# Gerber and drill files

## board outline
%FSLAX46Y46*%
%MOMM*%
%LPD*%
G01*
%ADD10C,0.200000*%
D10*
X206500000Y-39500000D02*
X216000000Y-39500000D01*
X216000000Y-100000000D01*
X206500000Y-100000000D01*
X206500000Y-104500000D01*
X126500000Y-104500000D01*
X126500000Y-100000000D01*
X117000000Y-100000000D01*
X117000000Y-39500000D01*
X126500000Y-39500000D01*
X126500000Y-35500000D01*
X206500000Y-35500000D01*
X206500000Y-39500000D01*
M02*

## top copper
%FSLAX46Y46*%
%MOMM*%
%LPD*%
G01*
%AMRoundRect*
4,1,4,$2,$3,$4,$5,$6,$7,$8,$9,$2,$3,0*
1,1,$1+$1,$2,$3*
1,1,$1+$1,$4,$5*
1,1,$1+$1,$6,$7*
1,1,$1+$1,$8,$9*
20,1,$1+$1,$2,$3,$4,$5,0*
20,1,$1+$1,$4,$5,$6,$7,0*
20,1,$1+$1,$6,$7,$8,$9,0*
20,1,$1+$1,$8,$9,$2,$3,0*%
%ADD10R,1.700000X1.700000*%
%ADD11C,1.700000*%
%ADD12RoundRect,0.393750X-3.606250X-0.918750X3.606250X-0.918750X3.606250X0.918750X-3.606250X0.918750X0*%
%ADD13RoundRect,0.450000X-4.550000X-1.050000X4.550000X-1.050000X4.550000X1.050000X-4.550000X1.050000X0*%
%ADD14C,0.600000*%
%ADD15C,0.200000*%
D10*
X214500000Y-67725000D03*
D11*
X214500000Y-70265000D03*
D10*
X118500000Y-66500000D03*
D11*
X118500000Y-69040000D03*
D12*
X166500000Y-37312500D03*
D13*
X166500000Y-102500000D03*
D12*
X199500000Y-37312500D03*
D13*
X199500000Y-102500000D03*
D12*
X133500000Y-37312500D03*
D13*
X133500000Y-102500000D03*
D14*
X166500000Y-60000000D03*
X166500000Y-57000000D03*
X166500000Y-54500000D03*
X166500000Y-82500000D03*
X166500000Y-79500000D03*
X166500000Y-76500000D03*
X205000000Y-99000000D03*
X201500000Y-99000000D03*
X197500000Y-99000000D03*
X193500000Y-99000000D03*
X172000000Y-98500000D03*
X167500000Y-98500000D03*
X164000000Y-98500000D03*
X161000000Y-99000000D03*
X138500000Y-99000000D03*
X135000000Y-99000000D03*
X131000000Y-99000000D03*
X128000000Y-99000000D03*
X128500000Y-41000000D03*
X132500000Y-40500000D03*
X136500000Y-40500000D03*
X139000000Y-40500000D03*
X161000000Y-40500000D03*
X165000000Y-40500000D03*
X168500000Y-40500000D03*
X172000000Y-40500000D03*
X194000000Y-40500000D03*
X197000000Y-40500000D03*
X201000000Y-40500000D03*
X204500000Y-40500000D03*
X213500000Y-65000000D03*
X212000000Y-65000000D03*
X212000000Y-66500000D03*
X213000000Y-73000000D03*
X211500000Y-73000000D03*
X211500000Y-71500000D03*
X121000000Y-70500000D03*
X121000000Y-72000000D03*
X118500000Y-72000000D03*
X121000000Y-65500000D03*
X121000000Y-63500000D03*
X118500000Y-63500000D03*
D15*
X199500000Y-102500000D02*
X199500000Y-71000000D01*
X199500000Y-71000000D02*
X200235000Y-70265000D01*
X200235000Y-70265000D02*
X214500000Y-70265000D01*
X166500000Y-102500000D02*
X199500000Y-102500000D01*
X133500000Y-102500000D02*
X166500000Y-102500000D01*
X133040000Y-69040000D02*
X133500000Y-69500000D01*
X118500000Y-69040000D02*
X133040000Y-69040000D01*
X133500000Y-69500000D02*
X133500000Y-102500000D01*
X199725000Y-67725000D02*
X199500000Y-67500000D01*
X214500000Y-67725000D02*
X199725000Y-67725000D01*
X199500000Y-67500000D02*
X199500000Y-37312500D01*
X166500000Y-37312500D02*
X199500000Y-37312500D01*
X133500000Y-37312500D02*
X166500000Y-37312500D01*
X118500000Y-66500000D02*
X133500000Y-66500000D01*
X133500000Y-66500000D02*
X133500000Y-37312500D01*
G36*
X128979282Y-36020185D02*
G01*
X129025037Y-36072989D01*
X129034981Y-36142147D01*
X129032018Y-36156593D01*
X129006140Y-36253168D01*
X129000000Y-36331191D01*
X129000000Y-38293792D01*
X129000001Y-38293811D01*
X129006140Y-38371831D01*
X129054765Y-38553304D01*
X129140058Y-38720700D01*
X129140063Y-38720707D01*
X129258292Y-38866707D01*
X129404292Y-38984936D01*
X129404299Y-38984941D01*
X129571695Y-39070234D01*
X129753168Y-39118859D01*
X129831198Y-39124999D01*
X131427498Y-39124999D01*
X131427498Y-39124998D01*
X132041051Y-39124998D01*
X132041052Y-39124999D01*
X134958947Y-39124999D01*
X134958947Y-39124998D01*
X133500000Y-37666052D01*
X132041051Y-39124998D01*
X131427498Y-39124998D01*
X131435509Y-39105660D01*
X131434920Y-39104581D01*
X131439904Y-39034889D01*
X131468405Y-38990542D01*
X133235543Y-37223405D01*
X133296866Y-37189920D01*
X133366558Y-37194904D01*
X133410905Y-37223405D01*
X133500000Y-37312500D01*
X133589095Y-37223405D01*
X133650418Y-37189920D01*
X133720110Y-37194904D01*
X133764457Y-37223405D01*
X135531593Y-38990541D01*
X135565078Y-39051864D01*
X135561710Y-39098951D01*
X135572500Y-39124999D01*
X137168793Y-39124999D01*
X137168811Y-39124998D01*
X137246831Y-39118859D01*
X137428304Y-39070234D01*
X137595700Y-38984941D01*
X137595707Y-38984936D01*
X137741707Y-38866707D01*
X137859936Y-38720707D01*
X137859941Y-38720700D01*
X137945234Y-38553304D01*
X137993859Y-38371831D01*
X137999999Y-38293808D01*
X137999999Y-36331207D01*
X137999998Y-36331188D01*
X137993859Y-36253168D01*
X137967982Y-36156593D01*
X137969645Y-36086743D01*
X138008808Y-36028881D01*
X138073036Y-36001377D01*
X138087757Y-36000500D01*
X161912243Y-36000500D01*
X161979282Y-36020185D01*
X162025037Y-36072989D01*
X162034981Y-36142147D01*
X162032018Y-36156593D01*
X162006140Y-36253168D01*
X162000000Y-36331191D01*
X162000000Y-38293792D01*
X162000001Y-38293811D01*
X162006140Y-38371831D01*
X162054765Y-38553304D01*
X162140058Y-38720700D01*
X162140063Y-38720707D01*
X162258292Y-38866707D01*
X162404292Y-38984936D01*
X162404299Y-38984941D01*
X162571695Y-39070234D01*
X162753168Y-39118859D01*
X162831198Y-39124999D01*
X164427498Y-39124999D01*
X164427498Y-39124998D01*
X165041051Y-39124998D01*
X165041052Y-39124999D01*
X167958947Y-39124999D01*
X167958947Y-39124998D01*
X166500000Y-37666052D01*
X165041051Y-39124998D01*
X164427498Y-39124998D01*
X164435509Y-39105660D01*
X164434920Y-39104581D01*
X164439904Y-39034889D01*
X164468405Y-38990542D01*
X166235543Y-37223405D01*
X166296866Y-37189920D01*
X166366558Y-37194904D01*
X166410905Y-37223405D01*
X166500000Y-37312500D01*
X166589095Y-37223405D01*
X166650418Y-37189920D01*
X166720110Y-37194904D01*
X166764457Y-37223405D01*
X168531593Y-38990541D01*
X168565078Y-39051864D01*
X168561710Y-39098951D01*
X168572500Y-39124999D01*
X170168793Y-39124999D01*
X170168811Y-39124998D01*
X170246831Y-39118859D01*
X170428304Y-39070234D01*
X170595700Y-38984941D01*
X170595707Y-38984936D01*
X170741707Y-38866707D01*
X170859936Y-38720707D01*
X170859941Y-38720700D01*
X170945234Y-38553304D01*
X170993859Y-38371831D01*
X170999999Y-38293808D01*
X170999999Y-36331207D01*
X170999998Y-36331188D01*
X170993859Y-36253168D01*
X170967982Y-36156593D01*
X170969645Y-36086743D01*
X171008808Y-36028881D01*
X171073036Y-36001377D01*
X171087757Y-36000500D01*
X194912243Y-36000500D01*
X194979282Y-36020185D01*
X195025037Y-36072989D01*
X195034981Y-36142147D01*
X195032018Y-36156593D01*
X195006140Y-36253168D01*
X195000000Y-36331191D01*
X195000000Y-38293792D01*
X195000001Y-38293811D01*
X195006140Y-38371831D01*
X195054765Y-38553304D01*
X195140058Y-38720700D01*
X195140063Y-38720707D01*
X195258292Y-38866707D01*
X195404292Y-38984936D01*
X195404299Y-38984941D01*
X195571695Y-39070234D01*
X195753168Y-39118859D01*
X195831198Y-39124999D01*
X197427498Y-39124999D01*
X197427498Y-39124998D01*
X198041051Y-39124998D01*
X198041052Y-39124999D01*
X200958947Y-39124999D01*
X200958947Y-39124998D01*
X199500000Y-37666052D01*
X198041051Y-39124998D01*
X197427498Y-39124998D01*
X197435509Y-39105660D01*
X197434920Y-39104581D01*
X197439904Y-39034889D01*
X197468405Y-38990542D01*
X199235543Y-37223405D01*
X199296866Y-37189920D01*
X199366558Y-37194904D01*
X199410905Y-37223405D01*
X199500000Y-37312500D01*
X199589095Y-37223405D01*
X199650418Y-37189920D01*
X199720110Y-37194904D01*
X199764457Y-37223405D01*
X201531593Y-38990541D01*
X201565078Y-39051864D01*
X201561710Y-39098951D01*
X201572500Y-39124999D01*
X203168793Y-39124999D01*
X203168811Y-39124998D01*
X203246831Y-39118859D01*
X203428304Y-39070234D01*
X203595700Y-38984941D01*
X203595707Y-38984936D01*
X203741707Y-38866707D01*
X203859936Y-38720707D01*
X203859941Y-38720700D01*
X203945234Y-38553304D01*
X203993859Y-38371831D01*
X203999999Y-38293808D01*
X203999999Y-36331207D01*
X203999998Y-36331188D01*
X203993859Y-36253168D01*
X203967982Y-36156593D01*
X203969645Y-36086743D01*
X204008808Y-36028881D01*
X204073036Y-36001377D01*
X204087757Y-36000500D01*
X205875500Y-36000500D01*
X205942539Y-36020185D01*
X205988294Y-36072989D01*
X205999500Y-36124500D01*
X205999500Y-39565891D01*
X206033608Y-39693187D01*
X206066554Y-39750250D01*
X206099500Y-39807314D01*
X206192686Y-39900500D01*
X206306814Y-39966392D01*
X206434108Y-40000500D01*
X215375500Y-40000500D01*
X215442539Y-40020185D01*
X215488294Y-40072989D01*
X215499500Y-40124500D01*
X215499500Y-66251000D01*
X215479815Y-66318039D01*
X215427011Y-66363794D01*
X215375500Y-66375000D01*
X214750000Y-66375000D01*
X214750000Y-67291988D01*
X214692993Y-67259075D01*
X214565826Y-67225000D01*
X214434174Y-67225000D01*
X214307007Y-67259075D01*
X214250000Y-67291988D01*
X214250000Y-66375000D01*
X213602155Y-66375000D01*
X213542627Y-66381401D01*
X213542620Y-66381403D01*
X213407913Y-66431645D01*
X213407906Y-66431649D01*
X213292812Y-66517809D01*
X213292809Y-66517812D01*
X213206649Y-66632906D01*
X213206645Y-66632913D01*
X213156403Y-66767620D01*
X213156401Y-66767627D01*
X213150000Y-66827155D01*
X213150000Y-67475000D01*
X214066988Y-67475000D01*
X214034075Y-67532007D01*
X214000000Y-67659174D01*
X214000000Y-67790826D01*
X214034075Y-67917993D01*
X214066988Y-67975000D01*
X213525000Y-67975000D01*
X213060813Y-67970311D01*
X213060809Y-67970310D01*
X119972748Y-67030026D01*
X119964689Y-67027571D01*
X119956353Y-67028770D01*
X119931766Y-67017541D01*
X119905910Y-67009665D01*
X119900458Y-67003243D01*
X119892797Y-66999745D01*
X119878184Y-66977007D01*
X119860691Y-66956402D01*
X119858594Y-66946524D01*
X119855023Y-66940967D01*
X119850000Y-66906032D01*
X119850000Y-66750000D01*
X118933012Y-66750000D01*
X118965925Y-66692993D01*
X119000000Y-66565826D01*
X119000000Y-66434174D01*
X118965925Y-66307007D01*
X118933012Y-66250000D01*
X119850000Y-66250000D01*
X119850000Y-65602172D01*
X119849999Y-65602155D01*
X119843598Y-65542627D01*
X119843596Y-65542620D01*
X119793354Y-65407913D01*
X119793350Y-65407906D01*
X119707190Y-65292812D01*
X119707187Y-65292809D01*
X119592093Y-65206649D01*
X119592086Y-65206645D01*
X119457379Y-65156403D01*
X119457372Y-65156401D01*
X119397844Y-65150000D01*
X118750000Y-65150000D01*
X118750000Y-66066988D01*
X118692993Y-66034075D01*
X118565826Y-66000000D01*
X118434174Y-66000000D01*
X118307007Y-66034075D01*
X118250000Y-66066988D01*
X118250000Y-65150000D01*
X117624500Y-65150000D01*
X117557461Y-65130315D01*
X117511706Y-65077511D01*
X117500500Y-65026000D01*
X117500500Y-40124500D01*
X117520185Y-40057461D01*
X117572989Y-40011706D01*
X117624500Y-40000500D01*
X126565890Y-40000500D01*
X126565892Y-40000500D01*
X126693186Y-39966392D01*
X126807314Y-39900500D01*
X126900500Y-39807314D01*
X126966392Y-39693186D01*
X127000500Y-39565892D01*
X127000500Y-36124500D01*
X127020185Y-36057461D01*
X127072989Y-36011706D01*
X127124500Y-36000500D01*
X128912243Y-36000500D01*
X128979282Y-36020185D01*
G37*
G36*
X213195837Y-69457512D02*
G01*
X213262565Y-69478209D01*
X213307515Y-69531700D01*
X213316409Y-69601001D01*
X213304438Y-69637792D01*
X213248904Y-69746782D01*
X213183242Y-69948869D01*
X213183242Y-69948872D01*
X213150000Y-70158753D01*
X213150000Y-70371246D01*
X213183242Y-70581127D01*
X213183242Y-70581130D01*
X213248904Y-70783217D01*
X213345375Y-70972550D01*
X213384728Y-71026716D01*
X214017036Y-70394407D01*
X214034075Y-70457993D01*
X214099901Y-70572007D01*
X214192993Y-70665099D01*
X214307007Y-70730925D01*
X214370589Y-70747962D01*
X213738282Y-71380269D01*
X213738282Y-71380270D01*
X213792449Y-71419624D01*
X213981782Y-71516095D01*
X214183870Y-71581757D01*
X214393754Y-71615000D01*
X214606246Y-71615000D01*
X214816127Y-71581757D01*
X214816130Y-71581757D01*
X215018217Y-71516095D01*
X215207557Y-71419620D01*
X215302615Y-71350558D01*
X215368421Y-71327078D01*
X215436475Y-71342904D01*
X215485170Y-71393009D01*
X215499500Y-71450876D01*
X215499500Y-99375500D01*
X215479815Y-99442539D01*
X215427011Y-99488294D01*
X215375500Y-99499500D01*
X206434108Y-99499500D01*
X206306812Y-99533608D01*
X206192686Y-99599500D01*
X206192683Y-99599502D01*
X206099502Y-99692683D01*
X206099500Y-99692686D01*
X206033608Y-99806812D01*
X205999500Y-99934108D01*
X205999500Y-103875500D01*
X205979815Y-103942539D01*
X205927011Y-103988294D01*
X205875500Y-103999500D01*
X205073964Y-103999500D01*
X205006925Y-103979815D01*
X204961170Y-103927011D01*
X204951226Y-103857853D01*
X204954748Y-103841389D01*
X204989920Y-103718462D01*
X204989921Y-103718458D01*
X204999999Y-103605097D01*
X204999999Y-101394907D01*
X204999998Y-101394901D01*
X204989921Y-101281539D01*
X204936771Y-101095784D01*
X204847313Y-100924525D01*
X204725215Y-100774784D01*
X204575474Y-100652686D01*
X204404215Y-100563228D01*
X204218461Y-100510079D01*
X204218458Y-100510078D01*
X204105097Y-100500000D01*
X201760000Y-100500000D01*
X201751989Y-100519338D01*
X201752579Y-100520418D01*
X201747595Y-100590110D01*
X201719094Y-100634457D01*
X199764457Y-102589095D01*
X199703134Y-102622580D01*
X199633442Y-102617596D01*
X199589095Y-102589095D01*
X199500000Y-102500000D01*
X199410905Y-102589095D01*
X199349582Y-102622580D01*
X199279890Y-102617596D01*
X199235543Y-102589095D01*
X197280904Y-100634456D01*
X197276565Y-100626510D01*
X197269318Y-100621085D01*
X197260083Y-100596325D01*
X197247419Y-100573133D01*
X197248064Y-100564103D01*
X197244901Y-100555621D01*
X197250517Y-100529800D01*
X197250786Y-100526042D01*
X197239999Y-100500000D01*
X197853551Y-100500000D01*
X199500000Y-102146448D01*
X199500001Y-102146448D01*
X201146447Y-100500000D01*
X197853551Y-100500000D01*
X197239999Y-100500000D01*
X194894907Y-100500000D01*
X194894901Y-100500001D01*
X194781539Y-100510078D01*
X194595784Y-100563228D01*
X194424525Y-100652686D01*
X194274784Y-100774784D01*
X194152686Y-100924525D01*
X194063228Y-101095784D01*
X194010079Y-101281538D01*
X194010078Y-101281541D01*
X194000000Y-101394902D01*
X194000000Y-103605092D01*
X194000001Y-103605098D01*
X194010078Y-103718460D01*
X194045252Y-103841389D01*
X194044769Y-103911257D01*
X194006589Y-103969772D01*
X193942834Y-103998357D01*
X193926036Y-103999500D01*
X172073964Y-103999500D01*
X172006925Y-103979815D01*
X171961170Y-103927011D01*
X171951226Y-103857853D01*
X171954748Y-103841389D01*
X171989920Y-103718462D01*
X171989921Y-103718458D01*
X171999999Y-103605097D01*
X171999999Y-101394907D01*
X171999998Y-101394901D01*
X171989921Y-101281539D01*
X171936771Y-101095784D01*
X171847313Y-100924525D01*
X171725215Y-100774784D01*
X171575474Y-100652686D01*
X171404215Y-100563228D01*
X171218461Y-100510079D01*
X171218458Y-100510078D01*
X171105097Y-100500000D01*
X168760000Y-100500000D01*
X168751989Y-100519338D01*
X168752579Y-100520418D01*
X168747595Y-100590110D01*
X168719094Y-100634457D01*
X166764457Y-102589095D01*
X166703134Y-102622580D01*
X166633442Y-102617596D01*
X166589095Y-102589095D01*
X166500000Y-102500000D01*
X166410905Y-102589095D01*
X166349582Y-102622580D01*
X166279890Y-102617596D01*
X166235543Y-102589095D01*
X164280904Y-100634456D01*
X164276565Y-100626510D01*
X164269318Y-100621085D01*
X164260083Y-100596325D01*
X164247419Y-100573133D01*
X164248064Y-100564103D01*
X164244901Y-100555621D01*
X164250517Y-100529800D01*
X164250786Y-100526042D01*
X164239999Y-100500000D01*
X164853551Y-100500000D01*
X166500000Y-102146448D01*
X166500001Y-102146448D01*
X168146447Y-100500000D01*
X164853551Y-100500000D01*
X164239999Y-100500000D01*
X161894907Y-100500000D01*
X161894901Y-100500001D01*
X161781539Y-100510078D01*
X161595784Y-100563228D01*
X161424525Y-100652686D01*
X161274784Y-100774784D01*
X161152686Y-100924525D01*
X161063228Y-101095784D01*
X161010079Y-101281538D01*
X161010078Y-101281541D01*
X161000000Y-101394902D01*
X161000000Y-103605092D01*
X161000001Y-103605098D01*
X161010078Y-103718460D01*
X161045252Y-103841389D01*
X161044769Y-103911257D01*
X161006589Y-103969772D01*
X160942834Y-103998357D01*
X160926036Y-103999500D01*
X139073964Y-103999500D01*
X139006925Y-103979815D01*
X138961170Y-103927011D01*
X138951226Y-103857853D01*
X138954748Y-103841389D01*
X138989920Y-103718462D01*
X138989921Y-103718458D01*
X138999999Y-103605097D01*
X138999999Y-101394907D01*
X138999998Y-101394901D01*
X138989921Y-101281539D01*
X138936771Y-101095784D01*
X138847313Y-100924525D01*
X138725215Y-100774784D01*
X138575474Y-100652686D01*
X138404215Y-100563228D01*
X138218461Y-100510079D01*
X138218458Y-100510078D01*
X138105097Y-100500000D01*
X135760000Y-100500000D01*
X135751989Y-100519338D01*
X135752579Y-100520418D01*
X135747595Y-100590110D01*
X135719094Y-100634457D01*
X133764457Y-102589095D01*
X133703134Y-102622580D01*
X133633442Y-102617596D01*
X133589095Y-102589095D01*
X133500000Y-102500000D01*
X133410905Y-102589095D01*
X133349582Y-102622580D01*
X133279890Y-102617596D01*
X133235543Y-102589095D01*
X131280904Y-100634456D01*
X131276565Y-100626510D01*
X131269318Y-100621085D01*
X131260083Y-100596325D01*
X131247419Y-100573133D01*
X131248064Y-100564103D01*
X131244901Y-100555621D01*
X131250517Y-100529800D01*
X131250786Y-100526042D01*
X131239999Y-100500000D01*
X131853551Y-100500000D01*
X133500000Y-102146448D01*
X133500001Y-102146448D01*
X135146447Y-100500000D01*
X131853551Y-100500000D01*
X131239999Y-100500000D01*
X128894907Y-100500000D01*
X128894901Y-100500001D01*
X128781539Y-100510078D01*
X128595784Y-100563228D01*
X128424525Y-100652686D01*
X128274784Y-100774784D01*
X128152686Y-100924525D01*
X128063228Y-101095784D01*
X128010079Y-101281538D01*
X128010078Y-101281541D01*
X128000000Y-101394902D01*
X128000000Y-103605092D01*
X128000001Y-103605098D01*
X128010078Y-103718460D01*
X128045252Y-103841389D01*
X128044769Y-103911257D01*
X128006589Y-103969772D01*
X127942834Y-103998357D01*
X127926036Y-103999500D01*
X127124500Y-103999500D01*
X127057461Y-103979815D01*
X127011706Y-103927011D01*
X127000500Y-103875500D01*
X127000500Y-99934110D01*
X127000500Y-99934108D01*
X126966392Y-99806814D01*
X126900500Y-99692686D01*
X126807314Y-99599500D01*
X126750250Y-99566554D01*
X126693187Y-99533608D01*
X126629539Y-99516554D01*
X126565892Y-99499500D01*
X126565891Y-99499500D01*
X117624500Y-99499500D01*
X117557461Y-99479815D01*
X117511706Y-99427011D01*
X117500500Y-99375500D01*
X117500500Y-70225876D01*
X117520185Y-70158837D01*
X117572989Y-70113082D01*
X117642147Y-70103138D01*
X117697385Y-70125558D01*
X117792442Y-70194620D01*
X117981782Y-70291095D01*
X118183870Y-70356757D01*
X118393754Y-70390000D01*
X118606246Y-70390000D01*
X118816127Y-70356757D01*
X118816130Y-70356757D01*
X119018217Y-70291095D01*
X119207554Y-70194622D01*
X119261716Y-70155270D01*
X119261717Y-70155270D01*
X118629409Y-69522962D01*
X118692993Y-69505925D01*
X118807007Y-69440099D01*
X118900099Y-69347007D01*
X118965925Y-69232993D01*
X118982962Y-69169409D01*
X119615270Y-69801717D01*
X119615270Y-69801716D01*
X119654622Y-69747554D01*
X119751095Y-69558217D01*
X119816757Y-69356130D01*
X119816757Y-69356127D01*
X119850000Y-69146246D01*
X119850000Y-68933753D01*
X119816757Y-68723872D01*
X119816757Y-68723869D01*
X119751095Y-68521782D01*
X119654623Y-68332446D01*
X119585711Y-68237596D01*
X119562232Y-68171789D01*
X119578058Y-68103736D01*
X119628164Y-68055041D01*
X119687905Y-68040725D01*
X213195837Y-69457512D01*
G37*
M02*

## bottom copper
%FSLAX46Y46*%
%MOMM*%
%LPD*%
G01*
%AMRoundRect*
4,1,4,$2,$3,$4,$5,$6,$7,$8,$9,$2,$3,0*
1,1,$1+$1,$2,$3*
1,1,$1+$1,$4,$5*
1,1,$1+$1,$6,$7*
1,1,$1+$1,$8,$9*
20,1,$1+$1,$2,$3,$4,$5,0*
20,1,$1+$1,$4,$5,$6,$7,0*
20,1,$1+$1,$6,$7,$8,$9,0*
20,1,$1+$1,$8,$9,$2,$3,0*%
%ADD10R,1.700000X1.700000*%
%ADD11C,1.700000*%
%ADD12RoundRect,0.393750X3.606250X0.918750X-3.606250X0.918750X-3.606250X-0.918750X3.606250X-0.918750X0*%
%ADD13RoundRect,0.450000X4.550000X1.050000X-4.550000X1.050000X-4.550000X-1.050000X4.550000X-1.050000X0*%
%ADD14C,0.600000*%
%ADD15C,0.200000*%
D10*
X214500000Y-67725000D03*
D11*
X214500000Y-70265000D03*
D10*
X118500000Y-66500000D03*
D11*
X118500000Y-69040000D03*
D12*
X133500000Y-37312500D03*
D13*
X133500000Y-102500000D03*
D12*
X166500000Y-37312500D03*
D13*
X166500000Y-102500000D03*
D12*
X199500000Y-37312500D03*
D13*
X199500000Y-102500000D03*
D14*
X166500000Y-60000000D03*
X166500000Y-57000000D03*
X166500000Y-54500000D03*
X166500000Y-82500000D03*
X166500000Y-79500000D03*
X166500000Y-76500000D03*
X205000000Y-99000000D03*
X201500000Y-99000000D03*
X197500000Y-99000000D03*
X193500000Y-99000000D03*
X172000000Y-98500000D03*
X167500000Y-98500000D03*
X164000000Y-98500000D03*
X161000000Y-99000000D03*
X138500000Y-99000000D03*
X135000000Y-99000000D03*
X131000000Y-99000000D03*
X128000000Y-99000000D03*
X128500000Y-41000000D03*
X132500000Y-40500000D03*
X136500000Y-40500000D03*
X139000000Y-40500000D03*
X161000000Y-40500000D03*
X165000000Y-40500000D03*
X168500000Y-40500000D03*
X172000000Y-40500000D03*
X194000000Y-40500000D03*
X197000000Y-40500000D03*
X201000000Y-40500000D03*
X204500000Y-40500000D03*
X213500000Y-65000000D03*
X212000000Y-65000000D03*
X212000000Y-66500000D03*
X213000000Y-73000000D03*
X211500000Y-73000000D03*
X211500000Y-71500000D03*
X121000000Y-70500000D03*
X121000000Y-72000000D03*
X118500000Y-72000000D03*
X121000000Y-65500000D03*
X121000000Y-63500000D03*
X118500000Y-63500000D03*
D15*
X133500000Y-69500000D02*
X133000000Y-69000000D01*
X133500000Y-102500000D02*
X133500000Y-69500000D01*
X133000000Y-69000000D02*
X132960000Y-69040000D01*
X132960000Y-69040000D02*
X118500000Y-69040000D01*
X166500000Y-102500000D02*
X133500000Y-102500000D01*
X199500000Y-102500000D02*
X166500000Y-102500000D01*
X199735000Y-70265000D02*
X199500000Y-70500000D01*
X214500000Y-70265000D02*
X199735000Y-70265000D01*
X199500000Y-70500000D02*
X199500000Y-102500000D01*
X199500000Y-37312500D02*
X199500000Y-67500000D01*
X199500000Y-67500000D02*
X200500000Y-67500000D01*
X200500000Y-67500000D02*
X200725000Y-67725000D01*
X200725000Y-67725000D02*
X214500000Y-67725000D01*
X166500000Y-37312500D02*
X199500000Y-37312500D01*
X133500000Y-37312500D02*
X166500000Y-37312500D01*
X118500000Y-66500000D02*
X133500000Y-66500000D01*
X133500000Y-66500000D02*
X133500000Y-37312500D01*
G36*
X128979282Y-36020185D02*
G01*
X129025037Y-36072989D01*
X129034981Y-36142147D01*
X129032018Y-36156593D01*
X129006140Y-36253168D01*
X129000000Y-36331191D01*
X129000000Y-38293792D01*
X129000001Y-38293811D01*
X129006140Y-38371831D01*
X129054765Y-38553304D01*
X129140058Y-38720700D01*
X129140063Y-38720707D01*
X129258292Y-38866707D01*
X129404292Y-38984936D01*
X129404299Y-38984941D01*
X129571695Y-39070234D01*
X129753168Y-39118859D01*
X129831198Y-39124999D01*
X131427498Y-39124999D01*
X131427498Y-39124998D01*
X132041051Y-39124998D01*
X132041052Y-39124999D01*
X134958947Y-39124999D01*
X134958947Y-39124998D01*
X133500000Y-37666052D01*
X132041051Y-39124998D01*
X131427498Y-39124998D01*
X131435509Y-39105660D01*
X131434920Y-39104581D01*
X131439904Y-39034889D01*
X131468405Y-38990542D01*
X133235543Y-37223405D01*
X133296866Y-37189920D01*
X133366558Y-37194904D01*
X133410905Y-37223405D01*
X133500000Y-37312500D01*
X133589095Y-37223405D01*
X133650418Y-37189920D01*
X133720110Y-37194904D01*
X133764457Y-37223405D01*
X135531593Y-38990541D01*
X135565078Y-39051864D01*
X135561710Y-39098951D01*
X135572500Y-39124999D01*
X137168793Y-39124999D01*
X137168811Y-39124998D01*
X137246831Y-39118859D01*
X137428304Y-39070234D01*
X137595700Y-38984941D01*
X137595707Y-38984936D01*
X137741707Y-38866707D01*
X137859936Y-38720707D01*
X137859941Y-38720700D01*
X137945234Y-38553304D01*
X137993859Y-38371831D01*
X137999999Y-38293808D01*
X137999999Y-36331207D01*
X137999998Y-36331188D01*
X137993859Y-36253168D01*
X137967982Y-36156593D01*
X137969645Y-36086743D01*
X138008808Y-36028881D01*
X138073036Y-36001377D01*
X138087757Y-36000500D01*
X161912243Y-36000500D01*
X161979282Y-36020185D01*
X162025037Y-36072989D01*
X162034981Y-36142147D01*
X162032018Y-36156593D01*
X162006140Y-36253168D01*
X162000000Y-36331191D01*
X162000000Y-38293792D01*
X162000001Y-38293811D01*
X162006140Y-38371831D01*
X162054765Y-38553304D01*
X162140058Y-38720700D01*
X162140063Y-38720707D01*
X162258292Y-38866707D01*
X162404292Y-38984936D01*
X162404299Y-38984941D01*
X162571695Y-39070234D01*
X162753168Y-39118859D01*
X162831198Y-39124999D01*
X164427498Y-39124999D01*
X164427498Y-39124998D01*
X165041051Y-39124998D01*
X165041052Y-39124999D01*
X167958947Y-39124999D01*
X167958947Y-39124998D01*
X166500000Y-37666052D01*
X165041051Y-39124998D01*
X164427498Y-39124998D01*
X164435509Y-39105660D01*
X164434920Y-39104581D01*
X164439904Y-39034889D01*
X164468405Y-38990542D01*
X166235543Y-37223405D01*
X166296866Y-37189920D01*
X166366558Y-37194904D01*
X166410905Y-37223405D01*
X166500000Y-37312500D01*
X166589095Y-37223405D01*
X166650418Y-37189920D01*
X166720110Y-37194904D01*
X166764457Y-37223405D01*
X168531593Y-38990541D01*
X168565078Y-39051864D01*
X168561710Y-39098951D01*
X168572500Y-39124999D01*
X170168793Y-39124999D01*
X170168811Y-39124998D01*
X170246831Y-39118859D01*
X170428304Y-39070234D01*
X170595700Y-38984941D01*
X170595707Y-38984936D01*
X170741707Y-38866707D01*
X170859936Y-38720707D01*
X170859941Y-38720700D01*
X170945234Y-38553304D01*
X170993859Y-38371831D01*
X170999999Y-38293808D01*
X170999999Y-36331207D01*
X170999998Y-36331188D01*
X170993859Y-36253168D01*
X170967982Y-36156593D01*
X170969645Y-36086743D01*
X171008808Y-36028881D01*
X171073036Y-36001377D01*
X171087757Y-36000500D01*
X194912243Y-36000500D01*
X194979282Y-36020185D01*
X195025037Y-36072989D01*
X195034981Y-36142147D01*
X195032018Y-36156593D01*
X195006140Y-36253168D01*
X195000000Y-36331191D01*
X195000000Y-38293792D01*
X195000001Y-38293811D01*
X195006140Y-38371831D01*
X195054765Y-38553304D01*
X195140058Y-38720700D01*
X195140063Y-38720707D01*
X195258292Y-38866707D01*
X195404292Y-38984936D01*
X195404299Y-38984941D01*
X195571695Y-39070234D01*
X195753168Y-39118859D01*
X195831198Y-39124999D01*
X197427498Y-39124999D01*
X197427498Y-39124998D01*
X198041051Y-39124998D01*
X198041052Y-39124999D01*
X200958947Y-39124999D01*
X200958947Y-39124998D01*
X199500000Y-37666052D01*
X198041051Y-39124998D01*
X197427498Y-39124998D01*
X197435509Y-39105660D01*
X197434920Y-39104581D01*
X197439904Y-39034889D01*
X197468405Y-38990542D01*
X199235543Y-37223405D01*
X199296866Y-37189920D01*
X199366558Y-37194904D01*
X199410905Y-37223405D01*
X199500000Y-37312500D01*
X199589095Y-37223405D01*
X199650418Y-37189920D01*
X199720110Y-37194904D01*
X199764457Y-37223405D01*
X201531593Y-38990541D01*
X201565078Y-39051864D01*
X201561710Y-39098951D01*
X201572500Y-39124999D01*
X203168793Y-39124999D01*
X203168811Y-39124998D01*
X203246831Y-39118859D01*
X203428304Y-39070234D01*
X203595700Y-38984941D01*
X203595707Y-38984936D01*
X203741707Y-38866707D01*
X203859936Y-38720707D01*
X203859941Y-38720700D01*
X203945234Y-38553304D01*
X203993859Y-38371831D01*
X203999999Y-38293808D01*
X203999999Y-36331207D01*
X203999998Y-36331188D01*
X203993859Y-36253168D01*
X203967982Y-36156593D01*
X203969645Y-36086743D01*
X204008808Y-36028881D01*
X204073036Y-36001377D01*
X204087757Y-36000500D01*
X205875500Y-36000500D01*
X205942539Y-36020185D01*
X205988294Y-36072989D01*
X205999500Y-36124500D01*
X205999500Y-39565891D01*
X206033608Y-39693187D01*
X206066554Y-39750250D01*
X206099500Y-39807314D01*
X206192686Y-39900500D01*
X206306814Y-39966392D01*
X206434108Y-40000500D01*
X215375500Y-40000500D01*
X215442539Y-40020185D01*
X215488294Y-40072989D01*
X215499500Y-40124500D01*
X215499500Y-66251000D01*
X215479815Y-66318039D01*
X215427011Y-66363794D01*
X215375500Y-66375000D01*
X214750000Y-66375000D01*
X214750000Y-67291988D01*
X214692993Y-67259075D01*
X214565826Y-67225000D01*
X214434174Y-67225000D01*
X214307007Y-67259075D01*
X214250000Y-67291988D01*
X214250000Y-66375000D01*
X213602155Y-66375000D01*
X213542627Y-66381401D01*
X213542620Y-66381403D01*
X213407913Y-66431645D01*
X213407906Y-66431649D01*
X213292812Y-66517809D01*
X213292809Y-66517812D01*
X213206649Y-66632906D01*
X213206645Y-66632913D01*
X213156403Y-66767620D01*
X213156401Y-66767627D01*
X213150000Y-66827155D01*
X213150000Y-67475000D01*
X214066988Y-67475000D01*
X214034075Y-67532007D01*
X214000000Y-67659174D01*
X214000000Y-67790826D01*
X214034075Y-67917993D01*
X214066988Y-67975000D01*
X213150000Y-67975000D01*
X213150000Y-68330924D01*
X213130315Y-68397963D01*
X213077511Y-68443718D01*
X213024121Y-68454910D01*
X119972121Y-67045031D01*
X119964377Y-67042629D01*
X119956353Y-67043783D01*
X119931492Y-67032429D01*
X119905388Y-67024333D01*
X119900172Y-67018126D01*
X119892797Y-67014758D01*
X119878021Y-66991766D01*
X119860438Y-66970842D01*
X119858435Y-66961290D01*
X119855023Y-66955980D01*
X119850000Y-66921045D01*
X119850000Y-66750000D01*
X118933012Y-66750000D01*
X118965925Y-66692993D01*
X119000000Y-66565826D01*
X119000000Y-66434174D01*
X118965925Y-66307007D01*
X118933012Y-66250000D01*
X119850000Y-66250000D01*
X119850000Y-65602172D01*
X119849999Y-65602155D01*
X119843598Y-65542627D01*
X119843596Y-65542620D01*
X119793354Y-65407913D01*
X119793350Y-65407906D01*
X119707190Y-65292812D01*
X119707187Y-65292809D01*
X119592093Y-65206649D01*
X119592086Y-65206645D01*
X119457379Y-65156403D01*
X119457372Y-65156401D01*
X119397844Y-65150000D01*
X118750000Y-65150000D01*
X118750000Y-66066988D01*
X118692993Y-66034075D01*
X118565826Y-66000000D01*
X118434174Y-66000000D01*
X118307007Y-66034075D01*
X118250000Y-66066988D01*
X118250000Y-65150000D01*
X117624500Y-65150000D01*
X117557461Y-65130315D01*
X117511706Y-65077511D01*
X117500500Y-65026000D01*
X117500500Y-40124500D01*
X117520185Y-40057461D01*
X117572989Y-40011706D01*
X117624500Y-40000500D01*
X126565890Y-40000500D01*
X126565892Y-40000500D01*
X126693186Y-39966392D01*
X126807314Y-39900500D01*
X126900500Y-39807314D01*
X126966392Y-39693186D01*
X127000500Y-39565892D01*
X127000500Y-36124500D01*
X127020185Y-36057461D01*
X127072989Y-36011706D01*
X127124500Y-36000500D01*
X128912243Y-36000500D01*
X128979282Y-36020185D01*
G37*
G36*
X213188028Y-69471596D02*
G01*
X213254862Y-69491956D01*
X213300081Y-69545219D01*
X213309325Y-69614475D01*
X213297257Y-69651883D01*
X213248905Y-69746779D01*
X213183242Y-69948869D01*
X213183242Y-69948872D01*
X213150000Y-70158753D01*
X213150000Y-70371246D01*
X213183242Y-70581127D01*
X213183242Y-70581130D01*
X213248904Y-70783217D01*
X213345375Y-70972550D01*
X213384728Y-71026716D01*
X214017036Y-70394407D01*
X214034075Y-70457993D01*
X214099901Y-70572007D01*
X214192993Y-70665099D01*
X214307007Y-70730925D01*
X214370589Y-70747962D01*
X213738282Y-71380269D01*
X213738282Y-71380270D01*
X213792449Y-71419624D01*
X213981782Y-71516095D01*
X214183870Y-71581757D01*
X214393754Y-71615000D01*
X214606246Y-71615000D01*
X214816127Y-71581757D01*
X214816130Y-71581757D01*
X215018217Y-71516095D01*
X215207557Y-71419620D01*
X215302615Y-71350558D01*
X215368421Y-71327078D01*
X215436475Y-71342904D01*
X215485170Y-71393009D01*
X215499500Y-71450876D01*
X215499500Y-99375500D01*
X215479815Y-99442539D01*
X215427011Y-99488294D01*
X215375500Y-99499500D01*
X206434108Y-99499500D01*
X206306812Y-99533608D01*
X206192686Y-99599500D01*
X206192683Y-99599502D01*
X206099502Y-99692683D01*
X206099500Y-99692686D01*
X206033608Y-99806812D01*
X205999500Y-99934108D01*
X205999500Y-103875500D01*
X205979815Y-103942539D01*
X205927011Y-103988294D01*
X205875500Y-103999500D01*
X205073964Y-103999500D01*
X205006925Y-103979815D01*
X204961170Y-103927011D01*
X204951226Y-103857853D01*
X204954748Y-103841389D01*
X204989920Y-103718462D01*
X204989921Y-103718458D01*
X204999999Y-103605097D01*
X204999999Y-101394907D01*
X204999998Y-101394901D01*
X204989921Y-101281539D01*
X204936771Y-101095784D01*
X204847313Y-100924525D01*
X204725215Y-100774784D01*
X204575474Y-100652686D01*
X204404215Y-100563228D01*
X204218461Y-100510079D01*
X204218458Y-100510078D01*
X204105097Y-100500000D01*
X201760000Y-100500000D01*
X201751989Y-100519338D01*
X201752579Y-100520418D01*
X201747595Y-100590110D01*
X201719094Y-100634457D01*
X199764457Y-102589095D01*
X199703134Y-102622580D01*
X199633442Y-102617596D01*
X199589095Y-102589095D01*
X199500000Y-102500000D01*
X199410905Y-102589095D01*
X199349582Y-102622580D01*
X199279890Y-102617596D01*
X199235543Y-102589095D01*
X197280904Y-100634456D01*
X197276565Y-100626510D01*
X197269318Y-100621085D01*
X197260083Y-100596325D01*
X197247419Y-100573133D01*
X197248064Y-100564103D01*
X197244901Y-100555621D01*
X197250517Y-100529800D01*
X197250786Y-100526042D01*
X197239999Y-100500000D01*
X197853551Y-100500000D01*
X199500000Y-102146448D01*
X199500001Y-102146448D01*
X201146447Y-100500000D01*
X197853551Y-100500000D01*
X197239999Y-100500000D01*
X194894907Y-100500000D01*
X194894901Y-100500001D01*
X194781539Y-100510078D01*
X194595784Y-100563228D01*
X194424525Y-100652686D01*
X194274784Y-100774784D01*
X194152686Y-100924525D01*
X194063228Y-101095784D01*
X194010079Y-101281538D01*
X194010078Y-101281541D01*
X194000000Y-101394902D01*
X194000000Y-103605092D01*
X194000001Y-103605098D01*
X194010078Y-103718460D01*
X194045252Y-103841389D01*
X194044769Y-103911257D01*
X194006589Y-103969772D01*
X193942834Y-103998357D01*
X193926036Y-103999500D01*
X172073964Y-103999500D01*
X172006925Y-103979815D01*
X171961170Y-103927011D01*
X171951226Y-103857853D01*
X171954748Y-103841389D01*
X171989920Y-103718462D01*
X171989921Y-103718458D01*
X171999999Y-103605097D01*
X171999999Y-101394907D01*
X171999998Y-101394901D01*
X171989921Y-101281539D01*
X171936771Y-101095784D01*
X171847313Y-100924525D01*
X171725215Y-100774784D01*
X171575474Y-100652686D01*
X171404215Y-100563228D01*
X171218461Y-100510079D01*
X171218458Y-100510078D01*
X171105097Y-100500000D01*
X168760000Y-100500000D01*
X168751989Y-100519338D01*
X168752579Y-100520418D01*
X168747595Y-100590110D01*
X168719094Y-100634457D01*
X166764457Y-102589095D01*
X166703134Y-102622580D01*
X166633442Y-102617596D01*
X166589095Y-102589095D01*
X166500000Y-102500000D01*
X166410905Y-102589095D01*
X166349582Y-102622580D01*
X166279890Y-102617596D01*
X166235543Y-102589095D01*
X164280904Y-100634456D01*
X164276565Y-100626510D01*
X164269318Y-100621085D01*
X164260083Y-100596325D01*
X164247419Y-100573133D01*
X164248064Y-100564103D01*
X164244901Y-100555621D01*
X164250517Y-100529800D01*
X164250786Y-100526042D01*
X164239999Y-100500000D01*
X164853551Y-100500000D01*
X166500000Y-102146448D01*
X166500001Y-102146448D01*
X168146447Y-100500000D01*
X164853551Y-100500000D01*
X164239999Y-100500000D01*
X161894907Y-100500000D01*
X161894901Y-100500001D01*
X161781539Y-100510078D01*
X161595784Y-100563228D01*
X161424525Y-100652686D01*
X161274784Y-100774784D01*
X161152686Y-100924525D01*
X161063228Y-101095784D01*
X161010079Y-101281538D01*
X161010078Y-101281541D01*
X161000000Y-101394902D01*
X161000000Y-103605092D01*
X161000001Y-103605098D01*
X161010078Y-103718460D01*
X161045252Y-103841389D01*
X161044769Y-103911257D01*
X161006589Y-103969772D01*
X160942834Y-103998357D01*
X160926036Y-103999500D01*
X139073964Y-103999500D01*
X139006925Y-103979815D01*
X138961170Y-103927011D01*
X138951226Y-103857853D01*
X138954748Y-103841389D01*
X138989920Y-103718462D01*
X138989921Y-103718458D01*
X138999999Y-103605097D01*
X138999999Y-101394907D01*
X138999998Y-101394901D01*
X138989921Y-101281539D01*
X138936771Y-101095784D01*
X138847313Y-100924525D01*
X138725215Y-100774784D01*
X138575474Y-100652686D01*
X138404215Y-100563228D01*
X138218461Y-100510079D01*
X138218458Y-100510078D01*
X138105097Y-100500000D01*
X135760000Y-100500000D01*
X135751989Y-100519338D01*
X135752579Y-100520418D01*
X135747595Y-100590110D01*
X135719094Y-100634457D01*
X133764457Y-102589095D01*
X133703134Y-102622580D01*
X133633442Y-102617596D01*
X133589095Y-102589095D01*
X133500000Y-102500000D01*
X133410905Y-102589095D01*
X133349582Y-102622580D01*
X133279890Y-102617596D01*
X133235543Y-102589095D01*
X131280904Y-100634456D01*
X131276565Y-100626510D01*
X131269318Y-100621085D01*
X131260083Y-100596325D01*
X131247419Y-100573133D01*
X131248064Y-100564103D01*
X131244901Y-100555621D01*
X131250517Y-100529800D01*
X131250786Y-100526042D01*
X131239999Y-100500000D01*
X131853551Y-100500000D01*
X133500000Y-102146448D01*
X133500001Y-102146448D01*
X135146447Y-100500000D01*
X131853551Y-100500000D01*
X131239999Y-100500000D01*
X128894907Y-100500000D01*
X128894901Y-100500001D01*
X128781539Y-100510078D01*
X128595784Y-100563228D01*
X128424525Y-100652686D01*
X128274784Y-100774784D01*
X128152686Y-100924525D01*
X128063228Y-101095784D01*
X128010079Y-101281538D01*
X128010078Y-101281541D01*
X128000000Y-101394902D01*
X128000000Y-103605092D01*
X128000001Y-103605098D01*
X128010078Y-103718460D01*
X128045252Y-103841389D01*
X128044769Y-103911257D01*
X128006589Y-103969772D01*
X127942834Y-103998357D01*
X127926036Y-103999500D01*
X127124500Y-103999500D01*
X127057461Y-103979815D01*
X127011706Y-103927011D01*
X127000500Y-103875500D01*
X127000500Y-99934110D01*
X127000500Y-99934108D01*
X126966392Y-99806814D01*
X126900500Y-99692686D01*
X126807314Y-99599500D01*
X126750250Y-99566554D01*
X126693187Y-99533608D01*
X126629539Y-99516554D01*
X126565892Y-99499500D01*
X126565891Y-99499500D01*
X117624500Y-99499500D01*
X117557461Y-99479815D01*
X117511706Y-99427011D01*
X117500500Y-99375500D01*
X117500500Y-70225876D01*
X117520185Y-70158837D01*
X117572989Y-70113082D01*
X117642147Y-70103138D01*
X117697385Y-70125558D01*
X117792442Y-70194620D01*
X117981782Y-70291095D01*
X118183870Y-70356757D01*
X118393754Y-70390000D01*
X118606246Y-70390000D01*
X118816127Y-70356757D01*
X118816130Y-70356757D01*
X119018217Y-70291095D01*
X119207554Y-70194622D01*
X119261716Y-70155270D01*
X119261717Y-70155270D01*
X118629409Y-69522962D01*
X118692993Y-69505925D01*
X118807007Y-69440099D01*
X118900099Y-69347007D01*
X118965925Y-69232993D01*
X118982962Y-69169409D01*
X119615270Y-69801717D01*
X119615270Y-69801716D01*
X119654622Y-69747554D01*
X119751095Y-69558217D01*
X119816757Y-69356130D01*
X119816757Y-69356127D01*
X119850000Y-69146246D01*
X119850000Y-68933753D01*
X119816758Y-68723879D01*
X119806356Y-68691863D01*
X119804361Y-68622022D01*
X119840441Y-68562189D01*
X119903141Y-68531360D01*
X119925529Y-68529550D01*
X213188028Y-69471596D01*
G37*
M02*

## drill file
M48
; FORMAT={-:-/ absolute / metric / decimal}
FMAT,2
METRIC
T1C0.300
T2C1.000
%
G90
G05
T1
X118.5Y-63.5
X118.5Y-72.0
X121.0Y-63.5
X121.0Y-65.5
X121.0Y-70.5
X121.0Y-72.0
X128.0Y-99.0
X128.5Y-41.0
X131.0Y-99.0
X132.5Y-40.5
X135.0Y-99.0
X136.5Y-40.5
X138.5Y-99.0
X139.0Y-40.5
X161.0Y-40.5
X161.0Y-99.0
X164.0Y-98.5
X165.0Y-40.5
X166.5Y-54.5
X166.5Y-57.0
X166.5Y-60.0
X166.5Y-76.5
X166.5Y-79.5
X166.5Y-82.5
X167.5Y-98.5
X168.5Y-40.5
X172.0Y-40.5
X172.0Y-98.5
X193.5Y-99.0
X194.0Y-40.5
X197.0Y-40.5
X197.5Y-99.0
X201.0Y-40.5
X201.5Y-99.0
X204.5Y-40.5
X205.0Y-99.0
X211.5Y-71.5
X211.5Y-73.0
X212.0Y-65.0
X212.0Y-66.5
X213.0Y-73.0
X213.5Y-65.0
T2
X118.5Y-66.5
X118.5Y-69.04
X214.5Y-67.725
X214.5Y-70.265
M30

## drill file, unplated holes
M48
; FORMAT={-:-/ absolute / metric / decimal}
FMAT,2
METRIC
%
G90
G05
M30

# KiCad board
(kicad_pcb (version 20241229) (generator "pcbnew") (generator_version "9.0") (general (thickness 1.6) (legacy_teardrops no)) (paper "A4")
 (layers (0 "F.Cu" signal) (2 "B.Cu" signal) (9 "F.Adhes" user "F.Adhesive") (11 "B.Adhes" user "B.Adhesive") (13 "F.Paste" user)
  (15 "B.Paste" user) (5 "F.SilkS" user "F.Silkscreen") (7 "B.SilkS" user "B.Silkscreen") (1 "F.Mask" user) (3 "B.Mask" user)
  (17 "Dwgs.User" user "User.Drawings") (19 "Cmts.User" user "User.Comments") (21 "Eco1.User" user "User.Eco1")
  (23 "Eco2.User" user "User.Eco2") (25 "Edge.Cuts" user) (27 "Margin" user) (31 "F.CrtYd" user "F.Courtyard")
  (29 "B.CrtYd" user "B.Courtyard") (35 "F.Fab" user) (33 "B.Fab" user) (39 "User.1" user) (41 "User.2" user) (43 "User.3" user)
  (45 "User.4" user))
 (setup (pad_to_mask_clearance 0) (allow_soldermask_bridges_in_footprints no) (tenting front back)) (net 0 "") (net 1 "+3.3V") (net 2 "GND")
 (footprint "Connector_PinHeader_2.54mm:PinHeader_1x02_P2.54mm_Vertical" (layer "F.Cu") (at 214.5 67.725)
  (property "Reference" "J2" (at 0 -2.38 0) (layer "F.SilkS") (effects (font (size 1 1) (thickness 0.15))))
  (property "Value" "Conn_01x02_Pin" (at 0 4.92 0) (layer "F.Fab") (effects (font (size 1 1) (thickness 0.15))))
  (pad "1" thru_hole rect (at 0 0) (size 1.7 1.7) (drill 1) (layers "*.Cu" "*.Mask") (remove_unused_layers no) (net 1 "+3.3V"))
  (pad "2" thru_hole circle (at 0 2.54) (size 1.7 1.7) (drill 1) (layers "*.Cu" "*.Mask") (remove_unused_layers no) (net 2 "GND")))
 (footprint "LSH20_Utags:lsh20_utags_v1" (layer "F.Cu") (at 166.5 70)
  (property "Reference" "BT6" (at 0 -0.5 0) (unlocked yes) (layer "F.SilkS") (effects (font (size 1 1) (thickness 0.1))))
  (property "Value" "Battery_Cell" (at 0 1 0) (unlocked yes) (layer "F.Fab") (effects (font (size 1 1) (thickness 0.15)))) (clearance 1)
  (pad "1" smd roundrect (at 0 -32.6875) (size 8 2.625) (layers "F.Cu" "F.Mask" "F.Paste") (roundrect_rratio 0.15) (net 1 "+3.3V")
   (thermal_bridge_angle 45))
  (pad "2" smd roundrect (at 0 32.5) (size 10 3) (layers "F.Cu" "F.Mask" "F.Paste") (roundrect_rratio 0.15) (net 2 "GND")
   (thermal_bridge_angle 45)))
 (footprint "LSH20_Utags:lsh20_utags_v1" (layer "F.Cu") (at 199.5 70)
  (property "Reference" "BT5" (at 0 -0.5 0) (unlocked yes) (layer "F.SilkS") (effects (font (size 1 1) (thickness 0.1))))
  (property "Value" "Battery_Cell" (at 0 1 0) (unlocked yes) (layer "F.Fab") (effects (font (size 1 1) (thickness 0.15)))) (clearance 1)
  (pad "1" smd roundrect (at 0 -32.6875) (size 8 2.625) (layers "F.Cu" "F.Mask" "F.Paste") (roundrect_rratio 0.15) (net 1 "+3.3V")
   (thermal_bridge_angle 45))
  (pad "2" smd roundrect (at 0 32.5) (size 10 3) (layers "F.Cu" "F.Mask" "F.Paste") (roundrect_rratio 0.15) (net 2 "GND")
   (thermal_bridge_angle 45)))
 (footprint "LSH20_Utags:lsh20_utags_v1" (layer "F.Cu") (at 133.5 70)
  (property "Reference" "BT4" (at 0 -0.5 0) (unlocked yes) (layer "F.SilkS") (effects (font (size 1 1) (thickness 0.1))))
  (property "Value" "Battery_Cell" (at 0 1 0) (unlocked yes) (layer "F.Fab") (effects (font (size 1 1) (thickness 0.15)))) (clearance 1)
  (pad "1" smd roundrect (at 0 -32.6875) (size 8 2.625) (layers "F.Cu" "F.Mask" "F.Paste") (roundrect_rratio 0.15) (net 1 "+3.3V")
   (thermal_bridge_angle 45))
  (pad "2" smd roundrect (at 0 32.5) (size 10 3) (layers "F.Cu" "F.Mask" "F.Paste") (roundrect_rratio 0.15) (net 2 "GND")
   (thermal_bridge_angle 45)))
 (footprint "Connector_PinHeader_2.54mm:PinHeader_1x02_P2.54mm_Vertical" (layer "F.Cu") (at 118.5 66.5)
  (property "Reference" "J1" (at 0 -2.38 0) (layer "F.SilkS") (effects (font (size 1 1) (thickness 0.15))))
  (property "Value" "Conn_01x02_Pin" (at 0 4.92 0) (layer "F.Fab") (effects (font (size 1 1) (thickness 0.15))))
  (pad "1" thru_hole rect (at 0 0) (size 1.7 1.7) (drill 1) (layers "*.Cu" "*.Mask") (remove_unused_layers no) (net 1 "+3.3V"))
  (pad "2" thru_hole circle (at 0 2.54) (size 1.7 1.7) (drill 1) (layers "*.Cu" "*.Mask") (remove_unused_layers no) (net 2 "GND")))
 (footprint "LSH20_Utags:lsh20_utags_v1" (layer "B.Cu") (at 166.5 70 180)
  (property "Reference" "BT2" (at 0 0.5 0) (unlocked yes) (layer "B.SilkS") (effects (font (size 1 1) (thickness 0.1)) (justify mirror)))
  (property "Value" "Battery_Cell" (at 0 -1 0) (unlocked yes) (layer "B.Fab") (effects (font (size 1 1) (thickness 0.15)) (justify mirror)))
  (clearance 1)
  (pad "1" smd roundrect (at 0 32.6875 180) (size 8 2.625) (layers "B.Cu" "B.Mask" "B.Paste") (roundrect_rratio 0.15) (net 1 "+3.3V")
   (thermal_bridge_angle 45))
  (pad "2" smd roundrect (at 0 -32.5 180) (size 10 3) (layers "B.Cu" "B.Mask" "B.Paste") (roundrect_rratio 0.15) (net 2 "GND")
   (thermal_bridge_angle 45)))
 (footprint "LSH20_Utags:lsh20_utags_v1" (layer "B.Cu") (at 199.5 70 180)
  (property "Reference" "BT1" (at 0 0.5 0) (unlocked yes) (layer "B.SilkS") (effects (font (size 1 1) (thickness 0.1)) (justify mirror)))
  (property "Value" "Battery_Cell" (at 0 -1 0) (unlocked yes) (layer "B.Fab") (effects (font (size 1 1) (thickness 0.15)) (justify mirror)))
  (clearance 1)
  (pad "1" smd roundrect (at 0 32.6875 180) (size 8 2.625) (layers "B.Cu" "B.Mask" "B.Paste") (roundrect_rratio 0.15) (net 1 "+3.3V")
   (thermal_bridge_angle 45))
  (pad "2" smd roundrect (at 0 -32.5 180) (size 10 3) (layers "B.Cu" "B.Mask" "B.Paste") (roundrect_rratio 0.15) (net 2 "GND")
   (thermal_bridge_angle 45)))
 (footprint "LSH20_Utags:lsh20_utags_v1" (layer "B.Cu") (at 133.5 70 180)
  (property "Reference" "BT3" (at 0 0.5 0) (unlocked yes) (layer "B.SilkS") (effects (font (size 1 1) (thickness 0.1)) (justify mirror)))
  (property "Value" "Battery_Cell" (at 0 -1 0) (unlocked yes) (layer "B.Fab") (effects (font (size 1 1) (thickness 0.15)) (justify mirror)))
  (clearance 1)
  (pad "1" smd roundrect (at 0 32.6875 180) (size 8 2.625) (layers "B.Cu" "B.Mask" "B.Paste") (roundrect_rratio 0.15) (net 1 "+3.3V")
   (thermal_bridge_angle 45))
  (pad "2" smd roundrect (at 0 -32.5 180) (size 10 3) (layers "B.Cu" "B.Mask" "B.Paste") (roundrect_rratio 0.15) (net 2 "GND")
   (thermal_bridge_angle 45)))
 (gr_poly
  (pts (xy 117 39.5) (xy 126.5 39.5) (xy 126.5 35.5) (xy 206.5 35.5) (xy 206.5 39.5) (xy 216 39.5) (xy 216 100) (xy 206.5 100)
   (xy 206.5 104.5) (xy 126.5 104.5) (xy 126.5 100) (xy 117 100))
  (stroke (width 0.2) (type solid)) (fill no) (layer "Edge.Cuts"))
 (segment (start 166.5 37.3125) (end 199.5 37.3125) (width 0.2) (layer "F.Cu") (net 1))
 (segment (start 133.5 37.3125) (end 166.5 37.3125) (width 0.2) (layer "F.Cu") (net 1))
 (segment (start 199.5 67.5) (end 199.5 37.3125) (width 0.2) (layer "F.Cu") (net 1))
 (segment (start 118.5 66.5) (end 133.5 66.5) (width 0.2) (layer "F.Cu") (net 1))
 (segment (start 133.5 66.5) (end 133.5 37.3125) (width 0.2) (layer "F.Cu") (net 1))
 (segment (start 214.5 67.725) (end 199.725 67.725) (width 0.2) (layer "F.Cu") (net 1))
 (segment (start 199.725 67.725) (end 199.5 67.5) (width 0.2) (layer "F.Cu") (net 1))
 (via (at 136.5 40.5) (size 0.6) (drill 0.3) (layers "F.Cu" "B.Cu") (free yes) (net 1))
 (via (at 165 40.5) (size 0.6) (drill 0.3) (layers "F.Cu" "B.Cu") (free yes) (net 1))
 (via (at 213.5 65) (size 0.6) (drill 0.3) (layers "F.Cu" "B.Cu") (free yes) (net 1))
 (via (at 197 40.5) (size 0.6) (drill 0.3) (layers "F.Cu" "B.Cu") (free yes) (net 1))
 (via (at 212 65) (size 0.6) (drill 0.3) (layers "F.Cu" "B.Cu") (free yes) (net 1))
 (via (at 168.5 40.5) (size 0.6) (drill 0.3) (layers "F.Cu" "B.Cu") (free yes) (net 1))
 (via (at 121 63.5) (size 0.6) (drill 0.3) (layers "F.Cu" "B.Cu") (free yes) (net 1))
 (via (at 172 40.5) (size 0.6) (drill 0.3) (layers "F.Cu" "B.Cu") (free yes) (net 1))
 (via (at 201 40.5) (size 0.6) (drill 0.3) (layers "F.Cu" "B.Cu") (free yes) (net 1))
 (via (at 166.5 60) (size 0.6) (drill 0.3) (layers "F.Cu" "B.Cu") (free yes) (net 1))
 (via (at 132.5 40.5) (size 0.6) (drill 0.3) (layers "F.Cu" "B.Cu") (free yes) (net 1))
 (via (at 166.5 57) (size 0.6) (drill 0.3) (layers "F.Cu" "B.Cu") (free yes) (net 1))
 (via (at 212 66.5) (size 0.6) (drill 0.3) (layers "F.Cu" "B.Cu") (free yes) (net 1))
 (via (at 194 40.5) (size 0.6) (drill 0.3) (layers "F.Cu" "B.Cu") (free yes) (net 1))
 (via (at 128.5 41) (size 0.6) (drill 0.3) (layers "F.Cu" "B.Cu") (free yes) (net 1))
 (via (at 204.5 40.5) (size 0.6) (drill 0.3) (layers "F.Cu" "B.Cu") (free yes) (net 1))
 (via (at 161 40.5) (size 0.6) (drill 0.3) (layers "F.Cu" "B.Cu") (free yes) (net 1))
 (via (at 139 40.5) (size 0.6) (drill 0.3) (layers "F.Cu" "B.Cu") (free yes) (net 1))
 (via (at 121 65.5) (size 0.6) (drill 0.3) (layers "F.Cu" "B.Cu") (free yes) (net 1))
 (via (at 118.5 63.5) (size 0.6) (drill 0.3) (layers "F.Cu" "B.Cu") (free yes) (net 1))
 (via (at 166.5 54.5) (size 0.6) (drill 0.3) (layers "F.Cu" "B.Cu") (free yes) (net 1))
 (segment (start 118.5 66.5) (end 133.5 66.5) (width 0.2) (layer "B.Cu") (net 1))
 (segment (start 199.5 67.5) (end 200.5 67.5) (width 0.2) (layer "B.Cu") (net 1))
 (segment (start 166.5 37.3125) (end 199.5 37.3125) (width 0.2) (layer "B.Cu") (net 1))
 (segment (start 133.5 66.5) (end 133.5 37.3125) (width 0.2) (layer "B.Cu") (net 1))
 (segment (start 133.5 37.3125) (end 166.5 37.3125) (width 0.2) (layer "B.Cu") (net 1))
 (segment (start 200.725 67.725) (end 214.5 67.725) (width 0.2) (layer "B.Cu") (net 1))
 (segment (start 199.5 37.3125) (end 199.5 67.5) (width 0.2) (layer "B.Cu") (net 1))
 (segment (start 200.5 67.5) (end 200.725 67.725) (width 0.2) (layer "B.Cu") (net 1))
 (segment (start 118.5 69.04) (end 133.04 69.04) (width 0.2) (layer "F.Cu") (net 2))
 (segment (start 133.04 69.04) (end 133.5 69.5) (width 0.2) (layer "F.Cu") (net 2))
 (segment (start 199.5 71) (end 200.235 70.265) (width 0.2) (layer "F.Cu") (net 2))
 (segment (start 200.235 70.265) (end 214.5 70.265) (width 0.2) (layer "F.Cu") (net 2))
 (segment (start 199.5 102.5) (end 199.5 71) (width 0.2) (layer "F.Cu") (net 2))
 (segment (start 166.5 102.5) (end 199.5 102.5) (width 0.2) (layer "F.Cu") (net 2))
 (segment (start 133.5 69.5) (end 133.5 102.5) (width 0.2) (layer "F.Cu") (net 2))
 (segment (start 133.5 102.5) (end 166.5 102.5) (width 0.2) (layer "F.Cu") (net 2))
 (via (at 166.5 82.5) (size 0.6) (drill 0.3) (layers "F.Cu" "B.Cu") (free yes) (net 2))
 (via (at 201.5 99) (size 0.6) (drill 0.3) (layers "F.Cu" "B.Cu") (free yes) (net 2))
 (via (at 121 70.5) (size 0.6) (drill 0.3) (layers "F.Cu" "B.Cu") (free yes) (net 2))
 (via (at 161 99) (size 0.6) (drill 0.3) (layers "F.Cu" "B.Cu") (free yes) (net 2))
 (via (at 211.5 73) (size 0.6) (drill 0.3) (layers "F.Cu" "B.Cu") (free yes) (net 2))
 (via (at 172 98.5) (size 0.6) (drill 0.3) (layers "F.Cu" "B.Cu") (free yes) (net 2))
 (via (at 211.5 71.5) (size 0.6) (drill 0.3) (layers "F.Cu" "B.Cu") (free yes) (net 2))
 (via (at 205 99) (size 0.6) (drill 0.3) (layers "F.Cu" "B.Cu") (free yes) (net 2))
 (via (at 121 72) (size 0.6) (drill 0.3) (layers "F.Cu" "B.Cu") (free yes) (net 2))
 (via (at 164 98.5) (size 0.6) (drill 0.3) (layers "F.Cu" "B.Cu") (free yes) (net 2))
 (via (at 118.5 72) (size 0.6) (drill 0.3) (layers "F.Cu" "B.Cu") (free yes) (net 2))
 (via (at 167.5 98.5) (size 0.6) (drill 0.3) (layers "F.Cu" "B.Cu") (free yes) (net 2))
 (via (at 138.5 99) (size 0.6) (drill 0.3) (layers "F.Cu" "B.Cu") (free yes) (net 2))
 (via (at 193.5 99) (size 0.6) (drill 0.3) (layers "F.Cu" "B.Cu") (free yes) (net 2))
 (via (at 213 73) (size 0.6) (drill 0.3) (layers "F.Cu" "B.Cu") (free yes) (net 2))
 (via (at 166.5 76.5) (size 0.6) (drill 0.3) (layers "F.Cu" "B.Cu") (free yes) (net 2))
 (via (at 135 99) (size 0.6) (drill 0.3) (layers "F.Cu" "B.Cu") (free yes) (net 2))
 (via (at 166.5 79.5) (size 0.6) (drill 0.3) (layers "F.Cu" "B.Cu") (free yes) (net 2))
 (via (at 197.5 99) (size 0.6) (drill 0.3) (layers "F.Cu" "B.Cu") (free yes) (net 2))
 (via (at 128 99) (size 0.6) (drill 0.3) (layers "F.Cu" "B.Cu") (free yes) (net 2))
 (via (at 131 99) (size 0.6) (drill 0.3) (layers "F.Cu" "B.Cu") (free yes) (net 2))
 (segment (start 214.5 70.265) (end 199.735 70.265) (width 0.2) (layer "B.Cu") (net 2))
 (segment (start 133.5 102.5) (end 133.5 69.5) (width 0.2) (layer "B.Cu") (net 2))
 (segment (start 166.5 102.5) (end 133.5 102.5) (width 0.2) (layer "B.Cu") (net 2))
 (segment (start 133 69) (end 132.96 69.04) (width 0.2) (layer "B.Cu") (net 2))
 (segment (start 199.735 70.265) (end 199.5 70.5) (width 0.2) (layer "B.Cu") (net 2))
 (segment (start 133.5 69.5) (end 133 69) (width 0.2) (layer "B.Cu") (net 2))
 (segment (start 132.96 69.04) (end 118.5 69.04) (width 0.2) (layer "B.Cu") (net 2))
 (segment (start 199.5 70.5) (end 199.5 102.5) (width 0.2) (layer "B.Cu") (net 2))
 (segment (start 199.5 102.5) (end 166.5 102.5) (width 0.2) (layer "B.Cu") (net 2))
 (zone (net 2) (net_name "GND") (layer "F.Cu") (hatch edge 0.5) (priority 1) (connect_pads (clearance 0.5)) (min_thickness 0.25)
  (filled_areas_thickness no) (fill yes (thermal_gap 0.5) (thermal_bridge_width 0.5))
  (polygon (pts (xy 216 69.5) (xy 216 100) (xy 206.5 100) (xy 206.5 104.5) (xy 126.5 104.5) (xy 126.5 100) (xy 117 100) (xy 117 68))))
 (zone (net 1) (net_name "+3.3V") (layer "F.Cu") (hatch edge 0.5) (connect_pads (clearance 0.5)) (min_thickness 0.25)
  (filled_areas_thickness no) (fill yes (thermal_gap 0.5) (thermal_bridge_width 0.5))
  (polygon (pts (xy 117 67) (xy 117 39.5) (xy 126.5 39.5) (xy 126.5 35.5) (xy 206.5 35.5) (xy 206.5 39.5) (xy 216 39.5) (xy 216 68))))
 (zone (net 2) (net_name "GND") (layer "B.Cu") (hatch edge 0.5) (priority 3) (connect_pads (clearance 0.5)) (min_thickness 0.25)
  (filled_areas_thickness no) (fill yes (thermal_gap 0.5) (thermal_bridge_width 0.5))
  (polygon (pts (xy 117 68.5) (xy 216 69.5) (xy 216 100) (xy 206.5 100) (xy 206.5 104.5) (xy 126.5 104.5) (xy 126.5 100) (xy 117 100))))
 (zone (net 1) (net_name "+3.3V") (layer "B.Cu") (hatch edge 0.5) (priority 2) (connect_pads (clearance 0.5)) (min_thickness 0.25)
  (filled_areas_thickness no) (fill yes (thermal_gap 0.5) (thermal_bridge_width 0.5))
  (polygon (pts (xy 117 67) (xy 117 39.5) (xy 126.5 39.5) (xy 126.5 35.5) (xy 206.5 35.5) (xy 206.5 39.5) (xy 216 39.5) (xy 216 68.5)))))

